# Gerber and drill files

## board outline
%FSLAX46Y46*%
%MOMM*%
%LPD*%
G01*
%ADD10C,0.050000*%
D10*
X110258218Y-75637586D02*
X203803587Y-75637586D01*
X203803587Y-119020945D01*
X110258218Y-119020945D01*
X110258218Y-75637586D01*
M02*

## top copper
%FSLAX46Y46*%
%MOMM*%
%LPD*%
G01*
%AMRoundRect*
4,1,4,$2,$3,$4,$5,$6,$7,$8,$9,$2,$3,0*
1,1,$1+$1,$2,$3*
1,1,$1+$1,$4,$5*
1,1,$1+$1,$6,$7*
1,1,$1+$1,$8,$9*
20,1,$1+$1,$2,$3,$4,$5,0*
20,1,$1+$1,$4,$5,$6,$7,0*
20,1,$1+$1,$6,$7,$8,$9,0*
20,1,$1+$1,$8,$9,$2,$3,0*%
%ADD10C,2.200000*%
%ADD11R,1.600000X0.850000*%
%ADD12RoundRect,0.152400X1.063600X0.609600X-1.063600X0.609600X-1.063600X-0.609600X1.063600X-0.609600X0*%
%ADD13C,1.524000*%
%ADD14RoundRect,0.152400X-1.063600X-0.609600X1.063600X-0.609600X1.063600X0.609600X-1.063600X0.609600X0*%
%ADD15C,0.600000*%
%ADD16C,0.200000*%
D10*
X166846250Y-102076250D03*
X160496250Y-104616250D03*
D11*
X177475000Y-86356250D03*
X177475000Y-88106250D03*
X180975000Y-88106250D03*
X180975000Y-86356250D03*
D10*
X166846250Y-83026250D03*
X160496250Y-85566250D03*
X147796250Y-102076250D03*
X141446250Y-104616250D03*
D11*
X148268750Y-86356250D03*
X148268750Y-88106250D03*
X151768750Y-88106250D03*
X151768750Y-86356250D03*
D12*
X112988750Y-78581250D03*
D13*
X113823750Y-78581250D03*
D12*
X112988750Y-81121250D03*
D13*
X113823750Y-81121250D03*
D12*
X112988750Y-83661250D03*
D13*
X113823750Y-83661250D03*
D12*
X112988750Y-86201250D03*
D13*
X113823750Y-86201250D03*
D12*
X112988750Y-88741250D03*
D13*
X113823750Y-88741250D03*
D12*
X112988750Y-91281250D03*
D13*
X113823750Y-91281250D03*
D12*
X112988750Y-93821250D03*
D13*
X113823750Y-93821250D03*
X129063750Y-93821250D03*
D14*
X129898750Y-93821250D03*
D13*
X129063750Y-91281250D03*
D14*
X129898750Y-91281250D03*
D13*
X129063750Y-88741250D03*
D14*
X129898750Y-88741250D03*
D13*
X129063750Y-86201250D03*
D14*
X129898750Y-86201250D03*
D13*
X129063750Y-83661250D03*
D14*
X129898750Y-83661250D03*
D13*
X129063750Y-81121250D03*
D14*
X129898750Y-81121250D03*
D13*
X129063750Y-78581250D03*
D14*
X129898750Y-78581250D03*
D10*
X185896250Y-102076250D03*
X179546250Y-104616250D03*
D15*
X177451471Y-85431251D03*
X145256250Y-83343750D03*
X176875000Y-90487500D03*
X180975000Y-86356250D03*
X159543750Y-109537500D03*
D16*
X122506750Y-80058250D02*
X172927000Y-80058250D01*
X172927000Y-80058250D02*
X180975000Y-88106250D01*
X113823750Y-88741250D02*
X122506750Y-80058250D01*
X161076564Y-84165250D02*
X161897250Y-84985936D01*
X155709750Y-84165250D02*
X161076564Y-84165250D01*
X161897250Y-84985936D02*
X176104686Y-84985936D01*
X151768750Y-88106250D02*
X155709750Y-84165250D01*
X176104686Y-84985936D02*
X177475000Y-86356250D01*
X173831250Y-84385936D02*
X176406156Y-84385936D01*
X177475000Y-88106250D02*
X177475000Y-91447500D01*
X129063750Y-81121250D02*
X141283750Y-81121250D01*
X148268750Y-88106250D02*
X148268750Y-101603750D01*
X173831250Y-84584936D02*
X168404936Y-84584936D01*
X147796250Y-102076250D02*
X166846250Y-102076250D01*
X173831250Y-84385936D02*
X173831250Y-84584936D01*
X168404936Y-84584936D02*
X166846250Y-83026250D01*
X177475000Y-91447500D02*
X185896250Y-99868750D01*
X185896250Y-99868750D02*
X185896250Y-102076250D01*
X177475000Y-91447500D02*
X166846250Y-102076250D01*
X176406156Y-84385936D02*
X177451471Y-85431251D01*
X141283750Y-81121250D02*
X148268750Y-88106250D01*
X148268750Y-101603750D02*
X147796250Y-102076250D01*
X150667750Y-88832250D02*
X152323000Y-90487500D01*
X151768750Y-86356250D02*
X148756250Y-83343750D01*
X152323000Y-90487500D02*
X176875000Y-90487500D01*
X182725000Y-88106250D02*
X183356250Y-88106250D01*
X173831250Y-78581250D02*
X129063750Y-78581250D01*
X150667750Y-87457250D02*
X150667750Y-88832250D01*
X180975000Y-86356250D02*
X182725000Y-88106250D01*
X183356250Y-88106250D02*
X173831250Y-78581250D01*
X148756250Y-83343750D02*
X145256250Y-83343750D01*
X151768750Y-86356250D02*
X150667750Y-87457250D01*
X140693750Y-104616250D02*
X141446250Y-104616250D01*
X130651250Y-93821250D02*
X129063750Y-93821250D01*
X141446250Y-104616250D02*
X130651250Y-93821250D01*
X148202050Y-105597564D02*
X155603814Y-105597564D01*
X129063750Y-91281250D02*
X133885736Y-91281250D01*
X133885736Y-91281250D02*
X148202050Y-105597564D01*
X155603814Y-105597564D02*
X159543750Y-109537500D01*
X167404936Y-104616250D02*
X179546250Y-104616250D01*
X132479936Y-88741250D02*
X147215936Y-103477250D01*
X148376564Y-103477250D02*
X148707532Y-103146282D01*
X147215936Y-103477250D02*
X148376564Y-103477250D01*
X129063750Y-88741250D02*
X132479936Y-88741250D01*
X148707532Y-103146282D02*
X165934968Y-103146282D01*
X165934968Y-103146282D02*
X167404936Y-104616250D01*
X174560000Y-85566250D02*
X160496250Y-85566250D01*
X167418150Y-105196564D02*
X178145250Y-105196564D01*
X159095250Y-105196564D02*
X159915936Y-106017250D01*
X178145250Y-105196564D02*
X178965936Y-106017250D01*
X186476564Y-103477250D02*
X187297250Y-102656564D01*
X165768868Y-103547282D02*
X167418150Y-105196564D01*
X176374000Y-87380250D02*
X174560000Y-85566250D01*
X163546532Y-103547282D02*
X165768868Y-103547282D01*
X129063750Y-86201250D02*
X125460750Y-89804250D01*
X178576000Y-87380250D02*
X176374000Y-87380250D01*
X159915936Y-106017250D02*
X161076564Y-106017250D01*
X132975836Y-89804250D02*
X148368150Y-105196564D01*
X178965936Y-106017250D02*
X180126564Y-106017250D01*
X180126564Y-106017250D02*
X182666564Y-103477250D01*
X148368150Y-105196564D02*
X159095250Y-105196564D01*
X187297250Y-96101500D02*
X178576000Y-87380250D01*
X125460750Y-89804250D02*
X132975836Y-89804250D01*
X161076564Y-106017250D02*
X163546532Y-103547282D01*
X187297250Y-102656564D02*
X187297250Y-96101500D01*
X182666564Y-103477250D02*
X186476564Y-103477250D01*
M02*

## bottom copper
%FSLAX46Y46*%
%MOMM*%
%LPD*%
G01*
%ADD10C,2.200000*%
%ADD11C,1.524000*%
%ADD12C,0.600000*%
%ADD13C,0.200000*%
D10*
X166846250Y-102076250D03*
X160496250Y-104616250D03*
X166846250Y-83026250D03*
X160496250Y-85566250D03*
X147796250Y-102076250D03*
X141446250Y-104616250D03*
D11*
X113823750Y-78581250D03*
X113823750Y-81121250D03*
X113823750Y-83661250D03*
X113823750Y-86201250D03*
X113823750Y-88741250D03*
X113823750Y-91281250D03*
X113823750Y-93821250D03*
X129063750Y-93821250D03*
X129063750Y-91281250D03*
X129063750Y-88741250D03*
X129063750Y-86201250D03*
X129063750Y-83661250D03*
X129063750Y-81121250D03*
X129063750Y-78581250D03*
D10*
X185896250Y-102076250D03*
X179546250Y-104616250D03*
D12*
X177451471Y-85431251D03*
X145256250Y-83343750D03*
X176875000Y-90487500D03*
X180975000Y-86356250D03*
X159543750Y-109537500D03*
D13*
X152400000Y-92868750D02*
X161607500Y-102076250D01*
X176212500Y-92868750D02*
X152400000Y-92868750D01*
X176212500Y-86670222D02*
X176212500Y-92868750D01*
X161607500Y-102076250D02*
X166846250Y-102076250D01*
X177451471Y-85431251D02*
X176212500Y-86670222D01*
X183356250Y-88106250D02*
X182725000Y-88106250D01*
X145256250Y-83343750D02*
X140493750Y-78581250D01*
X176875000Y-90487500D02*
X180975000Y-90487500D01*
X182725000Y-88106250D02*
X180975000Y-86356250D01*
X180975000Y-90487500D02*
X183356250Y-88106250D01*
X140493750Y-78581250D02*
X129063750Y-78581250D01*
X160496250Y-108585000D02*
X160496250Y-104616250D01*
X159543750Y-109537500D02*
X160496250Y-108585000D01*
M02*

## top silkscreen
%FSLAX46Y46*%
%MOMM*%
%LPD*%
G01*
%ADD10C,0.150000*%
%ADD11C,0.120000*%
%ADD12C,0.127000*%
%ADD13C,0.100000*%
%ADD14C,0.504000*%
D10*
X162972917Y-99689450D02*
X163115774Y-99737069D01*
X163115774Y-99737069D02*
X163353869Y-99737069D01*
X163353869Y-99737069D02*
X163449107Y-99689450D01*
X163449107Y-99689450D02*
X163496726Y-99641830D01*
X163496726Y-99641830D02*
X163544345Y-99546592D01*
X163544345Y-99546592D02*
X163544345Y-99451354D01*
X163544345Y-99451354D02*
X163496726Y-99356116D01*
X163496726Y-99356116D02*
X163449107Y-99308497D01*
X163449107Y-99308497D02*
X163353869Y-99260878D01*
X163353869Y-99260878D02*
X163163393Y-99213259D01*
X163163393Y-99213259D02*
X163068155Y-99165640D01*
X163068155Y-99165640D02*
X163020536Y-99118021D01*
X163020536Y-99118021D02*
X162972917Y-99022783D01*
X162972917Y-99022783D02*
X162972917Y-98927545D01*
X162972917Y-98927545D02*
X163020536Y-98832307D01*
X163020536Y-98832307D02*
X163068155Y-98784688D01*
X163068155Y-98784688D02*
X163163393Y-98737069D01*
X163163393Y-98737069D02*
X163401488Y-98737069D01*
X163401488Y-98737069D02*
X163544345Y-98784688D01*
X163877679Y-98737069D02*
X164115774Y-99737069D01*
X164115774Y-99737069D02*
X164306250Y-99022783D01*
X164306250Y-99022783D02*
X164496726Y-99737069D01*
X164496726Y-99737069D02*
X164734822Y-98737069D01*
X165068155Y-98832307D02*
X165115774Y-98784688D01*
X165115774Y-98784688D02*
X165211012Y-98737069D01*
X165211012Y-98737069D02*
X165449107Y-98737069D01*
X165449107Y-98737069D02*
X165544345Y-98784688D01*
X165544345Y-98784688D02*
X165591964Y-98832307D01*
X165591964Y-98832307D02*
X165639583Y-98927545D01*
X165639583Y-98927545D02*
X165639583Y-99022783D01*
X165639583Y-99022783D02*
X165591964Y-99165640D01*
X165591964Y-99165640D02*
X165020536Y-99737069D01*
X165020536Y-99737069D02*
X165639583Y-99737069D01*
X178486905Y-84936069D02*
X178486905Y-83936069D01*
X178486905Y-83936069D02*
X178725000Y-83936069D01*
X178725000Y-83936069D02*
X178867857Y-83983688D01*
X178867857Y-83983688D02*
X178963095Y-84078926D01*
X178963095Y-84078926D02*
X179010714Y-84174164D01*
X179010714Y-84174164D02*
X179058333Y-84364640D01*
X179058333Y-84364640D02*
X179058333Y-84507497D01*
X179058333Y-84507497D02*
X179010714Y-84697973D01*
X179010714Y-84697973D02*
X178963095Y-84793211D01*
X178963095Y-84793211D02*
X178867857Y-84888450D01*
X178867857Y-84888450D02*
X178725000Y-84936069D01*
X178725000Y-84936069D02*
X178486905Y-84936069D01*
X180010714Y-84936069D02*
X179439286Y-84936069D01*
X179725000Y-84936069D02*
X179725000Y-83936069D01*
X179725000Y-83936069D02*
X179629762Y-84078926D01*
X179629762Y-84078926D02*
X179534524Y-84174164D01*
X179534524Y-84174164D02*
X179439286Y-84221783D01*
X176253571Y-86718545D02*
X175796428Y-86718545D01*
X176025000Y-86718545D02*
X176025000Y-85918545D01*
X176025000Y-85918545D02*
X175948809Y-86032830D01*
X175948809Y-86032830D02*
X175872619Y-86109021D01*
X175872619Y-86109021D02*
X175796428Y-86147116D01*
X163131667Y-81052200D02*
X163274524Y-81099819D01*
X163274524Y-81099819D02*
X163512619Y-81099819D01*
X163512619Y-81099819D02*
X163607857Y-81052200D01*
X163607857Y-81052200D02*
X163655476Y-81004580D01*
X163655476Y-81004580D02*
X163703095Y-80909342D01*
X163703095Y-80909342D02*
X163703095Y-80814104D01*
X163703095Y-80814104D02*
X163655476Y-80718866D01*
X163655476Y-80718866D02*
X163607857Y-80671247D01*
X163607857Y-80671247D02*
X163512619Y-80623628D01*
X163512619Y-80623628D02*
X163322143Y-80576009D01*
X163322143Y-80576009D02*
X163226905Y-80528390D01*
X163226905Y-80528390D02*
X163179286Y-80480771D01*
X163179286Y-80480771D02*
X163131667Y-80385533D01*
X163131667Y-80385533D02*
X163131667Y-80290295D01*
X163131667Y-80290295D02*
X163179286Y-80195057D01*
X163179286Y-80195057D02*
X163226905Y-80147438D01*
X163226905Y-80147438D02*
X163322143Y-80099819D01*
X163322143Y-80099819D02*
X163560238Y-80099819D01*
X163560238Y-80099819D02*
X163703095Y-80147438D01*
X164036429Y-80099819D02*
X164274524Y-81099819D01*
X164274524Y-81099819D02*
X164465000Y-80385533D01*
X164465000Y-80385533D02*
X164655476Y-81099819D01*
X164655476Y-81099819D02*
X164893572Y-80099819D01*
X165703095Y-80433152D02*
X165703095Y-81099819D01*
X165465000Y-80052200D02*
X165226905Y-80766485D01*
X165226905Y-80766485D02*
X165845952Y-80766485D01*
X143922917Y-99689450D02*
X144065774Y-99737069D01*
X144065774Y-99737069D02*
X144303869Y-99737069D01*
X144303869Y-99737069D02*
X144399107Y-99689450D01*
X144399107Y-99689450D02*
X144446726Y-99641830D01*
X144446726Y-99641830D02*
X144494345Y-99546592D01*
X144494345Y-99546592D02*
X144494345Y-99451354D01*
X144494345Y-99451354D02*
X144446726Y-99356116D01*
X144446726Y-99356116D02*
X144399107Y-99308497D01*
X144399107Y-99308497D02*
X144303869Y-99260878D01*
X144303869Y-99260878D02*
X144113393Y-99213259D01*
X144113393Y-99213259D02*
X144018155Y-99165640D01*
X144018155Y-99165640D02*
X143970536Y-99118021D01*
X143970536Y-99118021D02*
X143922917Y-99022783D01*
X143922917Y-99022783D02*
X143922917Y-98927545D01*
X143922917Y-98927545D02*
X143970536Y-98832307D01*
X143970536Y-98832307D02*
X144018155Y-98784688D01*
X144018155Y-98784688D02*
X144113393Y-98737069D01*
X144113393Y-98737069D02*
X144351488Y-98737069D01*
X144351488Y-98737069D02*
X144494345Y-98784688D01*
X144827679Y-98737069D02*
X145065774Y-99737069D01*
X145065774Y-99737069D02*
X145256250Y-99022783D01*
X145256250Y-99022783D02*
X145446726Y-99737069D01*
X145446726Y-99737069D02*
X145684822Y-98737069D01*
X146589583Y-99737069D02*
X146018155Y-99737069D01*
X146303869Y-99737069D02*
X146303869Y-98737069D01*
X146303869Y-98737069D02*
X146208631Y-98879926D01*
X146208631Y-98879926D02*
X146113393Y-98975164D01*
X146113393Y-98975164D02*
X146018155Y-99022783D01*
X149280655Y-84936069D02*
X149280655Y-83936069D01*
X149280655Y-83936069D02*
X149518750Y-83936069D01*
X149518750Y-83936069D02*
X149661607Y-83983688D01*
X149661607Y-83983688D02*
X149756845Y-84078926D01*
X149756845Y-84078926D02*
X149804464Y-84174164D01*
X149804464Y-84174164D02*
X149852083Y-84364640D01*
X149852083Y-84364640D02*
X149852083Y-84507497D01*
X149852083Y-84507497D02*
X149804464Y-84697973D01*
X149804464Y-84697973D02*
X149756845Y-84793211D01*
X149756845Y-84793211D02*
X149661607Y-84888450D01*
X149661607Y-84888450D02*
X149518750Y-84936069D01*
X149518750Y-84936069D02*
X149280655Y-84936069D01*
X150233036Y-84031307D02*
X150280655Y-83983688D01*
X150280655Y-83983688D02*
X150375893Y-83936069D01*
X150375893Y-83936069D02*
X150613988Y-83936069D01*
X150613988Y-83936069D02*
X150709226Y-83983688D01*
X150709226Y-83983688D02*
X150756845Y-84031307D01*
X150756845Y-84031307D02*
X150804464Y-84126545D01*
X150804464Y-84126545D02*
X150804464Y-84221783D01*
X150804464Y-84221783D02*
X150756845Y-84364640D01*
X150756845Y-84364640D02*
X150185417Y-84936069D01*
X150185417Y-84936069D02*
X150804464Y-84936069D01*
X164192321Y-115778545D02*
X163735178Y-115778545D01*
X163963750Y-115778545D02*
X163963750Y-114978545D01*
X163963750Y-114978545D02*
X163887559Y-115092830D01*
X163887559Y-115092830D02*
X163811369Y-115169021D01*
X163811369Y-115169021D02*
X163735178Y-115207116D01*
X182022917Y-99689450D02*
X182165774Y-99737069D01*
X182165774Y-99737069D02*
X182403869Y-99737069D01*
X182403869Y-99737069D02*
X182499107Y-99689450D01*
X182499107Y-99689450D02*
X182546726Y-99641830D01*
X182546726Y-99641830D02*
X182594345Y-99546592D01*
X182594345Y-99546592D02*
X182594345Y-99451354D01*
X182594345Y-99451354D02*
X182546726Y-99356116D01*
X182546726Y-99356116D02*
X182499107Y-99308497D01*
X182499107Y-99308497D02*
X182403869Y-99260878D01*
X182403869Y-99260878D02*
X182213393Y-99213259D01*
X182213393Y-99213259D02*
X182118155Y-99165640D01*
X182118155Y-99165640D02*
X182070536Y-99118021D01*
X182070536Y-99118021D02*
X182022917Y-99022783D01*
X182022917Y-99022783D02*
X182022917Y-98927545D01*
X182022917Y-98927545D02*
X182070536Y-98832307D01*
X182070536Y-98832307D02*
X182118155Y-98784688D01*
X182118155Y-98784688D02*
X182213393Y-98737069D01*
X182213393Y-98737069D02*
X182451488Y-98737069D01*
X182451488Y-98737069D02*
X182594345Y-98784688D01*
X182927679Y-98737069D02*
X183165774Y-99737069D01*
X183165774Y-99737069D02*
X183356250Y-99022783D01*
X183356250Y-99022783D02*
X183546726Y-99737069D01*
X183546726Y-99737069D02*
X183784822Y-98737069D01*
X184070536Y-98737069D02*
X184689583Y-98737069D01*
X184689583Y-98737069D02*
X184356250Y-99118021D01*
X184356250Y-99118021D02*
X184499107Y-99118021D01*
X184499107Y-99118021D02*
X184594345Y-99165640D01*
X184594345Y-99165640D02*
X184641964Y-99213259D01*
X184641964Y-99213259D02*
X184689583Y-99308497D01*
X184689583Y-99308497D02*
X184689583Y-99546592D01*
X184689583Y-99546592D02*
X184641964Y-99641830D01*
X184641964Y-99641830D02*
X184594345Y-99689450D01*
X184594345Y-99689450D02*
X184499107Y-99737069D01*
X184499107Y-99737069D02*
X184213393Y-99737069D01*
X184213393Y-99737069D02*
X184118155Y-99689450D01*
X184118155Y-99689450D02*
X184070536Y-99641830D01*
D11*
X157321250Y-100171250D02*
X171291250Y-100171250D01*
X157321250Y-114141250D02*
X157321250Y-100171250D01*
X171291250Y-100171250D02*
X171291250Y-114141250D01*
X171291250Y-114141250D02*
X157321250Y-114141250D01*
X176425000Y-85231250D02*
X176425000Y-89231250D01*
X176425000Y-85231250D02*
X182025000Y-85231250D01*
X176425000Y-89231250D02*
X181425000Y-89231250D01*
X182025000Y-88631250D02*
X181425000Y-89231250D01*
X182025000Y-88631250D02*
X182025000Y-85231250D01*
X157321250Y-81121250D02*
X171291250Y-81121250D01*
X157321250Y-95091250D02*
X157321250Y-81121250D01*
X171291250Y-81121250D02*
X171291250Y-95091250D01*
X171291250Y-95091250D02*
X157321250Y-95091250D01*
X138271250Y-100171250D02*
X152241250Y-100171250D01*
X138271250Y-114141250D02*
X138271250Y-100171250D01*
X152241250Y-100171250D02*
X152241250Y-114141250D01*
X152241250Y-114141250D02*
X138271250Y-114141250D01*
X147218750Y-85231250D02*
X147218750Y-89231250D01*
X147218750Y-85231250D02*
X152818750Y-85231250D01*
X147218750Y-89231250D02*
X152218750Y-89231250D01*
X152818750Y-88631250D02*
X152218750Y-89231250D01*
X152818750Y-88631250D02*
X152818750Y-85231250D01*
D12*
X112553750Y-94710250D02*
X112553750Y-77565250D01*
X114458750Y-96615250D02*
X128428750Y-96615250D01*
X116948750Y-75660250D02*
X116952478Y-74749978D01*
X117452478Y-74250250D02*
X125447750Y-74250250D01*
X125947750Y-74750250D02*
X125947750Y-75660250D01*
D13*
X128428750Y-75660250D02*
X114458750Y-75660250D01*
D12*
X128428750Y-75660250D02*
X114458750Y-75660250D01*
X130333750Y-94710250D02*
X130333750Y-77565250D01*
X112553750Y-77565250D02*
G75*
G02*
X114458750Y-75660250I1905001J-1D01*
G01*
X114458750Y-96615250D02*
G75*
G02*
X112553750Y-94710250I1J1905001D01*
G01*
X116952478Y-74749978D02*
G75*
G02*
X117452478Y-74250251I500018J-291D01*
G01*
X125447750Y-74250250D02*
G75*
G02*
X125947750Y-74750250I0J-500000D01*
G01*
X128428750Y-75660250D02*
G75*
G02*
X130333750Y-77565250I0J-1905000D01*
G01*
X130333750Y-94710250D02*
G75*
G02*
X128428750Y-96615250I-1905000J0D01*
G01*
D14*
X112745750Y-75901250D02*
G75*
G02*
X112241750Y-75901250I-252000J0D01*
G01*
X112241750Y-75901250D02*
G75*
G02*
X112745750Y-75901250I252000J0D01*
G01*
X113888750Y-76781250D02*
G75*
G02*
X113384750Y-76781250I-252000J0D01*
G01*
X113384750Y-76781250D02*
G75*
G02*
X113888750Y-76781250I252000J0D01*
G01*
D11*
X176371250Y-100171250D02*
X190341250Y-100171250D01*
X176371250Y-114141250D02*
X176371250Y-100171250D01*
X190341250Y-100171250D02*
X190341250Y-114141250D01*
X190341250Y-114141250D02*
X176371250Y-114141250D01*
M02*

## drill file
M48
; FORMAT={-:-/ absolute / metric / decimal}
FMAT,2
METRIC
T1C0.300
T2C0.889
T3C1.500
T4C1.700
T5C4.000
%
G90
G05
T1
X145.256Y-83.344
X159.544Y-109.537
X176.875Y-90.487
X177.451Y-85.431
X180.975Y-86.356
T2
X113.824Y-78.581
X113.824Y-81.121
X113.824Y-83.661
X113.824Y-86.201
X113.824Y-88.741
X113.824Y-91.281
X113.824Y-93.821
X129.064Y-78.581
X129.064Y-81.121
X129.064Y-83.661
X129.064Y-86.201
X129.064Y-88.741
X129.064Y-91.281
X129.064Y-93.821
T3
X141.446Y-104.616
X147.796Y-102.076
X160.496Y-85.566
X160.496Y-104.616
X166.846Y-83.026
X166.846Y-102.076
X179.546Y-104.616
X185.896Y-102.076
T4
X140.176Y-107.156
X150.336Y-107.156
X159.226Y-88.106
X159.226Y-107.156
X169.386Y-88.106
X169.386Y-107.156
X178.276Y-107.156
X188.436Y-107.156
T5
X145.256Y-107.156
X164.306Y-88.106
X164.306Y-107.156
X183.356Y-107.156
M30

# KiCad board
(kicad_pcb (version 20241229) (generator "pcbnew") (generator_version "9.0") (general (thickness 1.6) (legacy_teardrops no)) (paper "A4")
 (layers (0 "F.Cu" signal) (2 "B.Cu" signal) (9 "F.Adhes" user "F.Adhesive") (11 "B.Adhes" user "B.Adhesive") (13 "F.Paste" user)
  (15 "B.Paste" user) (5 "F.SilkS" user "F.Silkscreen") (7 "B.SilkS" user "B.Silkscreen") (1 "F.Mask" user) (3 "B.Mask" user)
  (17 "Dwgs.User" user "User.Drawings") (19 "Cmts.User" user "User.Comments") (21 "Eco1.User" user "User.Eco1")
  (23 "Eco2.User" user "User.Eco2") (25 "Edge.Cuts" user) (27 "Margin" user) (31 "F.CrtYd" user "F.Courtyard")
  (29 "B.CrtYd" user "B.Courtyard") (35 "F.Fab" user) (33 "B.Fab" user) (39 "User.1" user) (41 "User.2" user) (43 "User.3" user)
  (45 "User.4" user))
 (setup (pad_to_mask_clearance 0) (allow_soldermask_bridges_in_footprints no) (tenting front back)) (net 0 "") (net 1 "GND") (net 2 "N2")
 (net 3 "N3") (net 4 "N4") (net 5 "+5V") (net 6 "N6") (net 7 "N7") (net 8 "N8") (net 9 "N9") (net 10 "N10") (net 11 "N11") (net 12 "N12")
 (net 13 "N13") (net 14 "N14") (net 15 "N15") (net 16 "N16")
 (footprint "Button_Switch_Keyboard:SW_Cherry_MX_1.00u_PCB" (layer "F.Cu") (at 166.84625 102.07625)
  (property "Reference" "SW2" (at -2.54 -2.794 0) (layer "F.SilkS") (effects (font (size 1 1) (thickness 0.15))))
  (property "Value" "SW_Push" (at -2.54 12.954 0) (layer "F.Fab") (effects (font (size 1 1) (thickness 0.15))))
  (fp_line (start -9.525 -1.905) (end 4.445 -1.905) (stroke (width 0.12) (type solid)) (layer "F.SilkS"))
  (fp_line (start -9.525 12.065) (end -9.525 -1.905) (stroke (width 0.12) (type solid)) (layer "F.SilkS"))
  (fp_line (start 4.445 -1.905) (end 4.445 12.065) (stroke (width 0.12) (type solid)) (layer "F.SilkS"))
  (fp_line (start 4.445 12.065) (end -9.525 12.065) (stroke (width 0.12) (type solid)) (layer "F.SilkS"))
  (pad "" np_thru_hole circle (at -7.62 5.08) (size 1.7 1.7) (drill 1.7) (layers "*.Cu" "*.Mask"))
  (pad "" np_thru_hole circle (at -2.54 5.08) (size 4 4) (drill 4) (layers "*.Cu" "*.Mask"))
  (pad "" np_thru_hole circle (at 2.54 5.08) (size 1.7 1.7) (drill 1.7) (layers "*.Cu" "*.Mask"))
  (pad "1" thru_hole circle (at 0 0) (size 2.2 2.2) (drill 1.5) (layers "*.Cu" "*.Mask") (remove_unused_layers no) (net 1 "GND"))
  (pad "2" thru_hole circle (at -6.35 2.54) (size 2.2 2.2) (drill 1.5) (layers "*.Cu" "*.Mask") (remove_unused_layers no) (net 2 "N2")))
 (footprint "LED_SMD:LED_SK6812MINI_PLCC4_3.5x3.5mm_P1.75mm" (layer "F.Cu") (at 179.225 87.23125)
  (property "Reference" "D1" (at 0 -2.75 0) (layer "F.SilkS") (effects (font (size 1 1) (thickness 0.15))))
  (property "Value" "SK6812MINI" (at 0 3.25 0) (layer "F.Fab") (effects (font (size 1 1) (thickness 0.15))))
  (fp_line (start -2.8 -2) (end -2.8 2) (stroke (width 0.12) (type default)) (layer "F.SilkS"))
  (fp_line (start -2.8 -2) (end 2.8 -2) (stroke (width 0.12) (type solid)) (layer "F.SilkS"))
  (fp_line (start -2.8 2) (end 2.2 2) (stroke (width 0.12) (type solid)) (layer "F.SilkS"))
  (fp_line (start 2.8 1.4) (end 2.2 2) (stroke (width 0.12) (type default)) (layer "F.SilkS"))
  (fp_line (start 2.8 1.4) (end 2.8 -2) (stroke (width 0.12) (type solid)) (layer "F.SilkS"))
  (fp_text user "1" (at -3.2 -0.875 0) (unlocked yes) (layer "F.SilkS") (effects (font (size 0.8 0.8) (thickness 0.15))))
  (pad "1" smd rect (at -1.75 -0.875) (size 1.6 0.85) (layers "F.Cu" "F.Mask" "F.Paste") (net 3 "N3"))
  (pad "2" smd rect (at -1.75 0.875) (size 1.6 0.85) (layers "F.Cu" "F.Mask" "F.Paste") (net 1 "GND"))
  (pad "3" smd rect (at 1.75 0.875) (size 1.6 0.85) (layers "F.Cu" "F.Mask" "F.Paste") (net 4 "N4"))
  (pad "4" smd rect (at 1.75 -0.875) (size 1.6 0.85) (layers "F.Cu" "F.Mask" "F.Paste") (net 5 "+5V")))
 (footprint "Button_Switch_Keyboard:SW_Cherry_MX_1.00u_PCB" (layer "F.Cu") (at 166.84625 83.02625)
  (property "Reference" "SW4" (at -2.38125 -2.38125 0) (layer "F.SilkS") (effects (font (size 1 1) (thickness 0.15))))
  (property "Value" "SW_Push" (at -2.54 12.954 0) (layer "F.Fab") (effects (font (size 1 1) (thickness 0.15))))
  (fp_line (start -9.525 -1.905) (end 4.445 -1.905) (stroke (width 0.12) (type solid)) (layer "F.SilkS"))
  (fp_line (start -9.525 12.065) (end -9.525 -1.905) (stroke (width 0.12) (type solid)) (layer "F.SilkS"))
  (fp_line (start 4.445 -1.905) (end 4.445 12.065) (stroke (width 0.12) (type solid)) (layer "F.SilkS"))
  (fp_line (start 4.445 12.065) (end -9.525 12.065) (stroke (width 0.12) (type solid)) (layer "F.SilkS"))
  (pad "" np_thru_hole circle (at -7.62 5.08) (size 1.7 1.7) (drill 1.7) (layers "*.Cu" "*.Mask"))
  (pad "" np_thru_hole circle (at -2.54 5.08) (size 4 4) (drill 4) (layers "*.Cu" "*.Mask"))
  (pad "" np_thru_hole circle (at 2.54 5.08) (size 1.7 1.7) (drill 1.7) (layers "*.Cu" "*.Mask"))
  (pad "1" thru_hole circle (at 0 0) (size 2.2 2.2) (drill 1.5) (layers "*.Cu" "*.Mask") (remove_unused_layers no) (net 1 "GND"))
  (pad "2" thru_hole circle (at -6.35 2.54) (size 2.2 2.2) (drill 1.5) (layers "*.Cu" "*.Mask") (remove_unused_layers no) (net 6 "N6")))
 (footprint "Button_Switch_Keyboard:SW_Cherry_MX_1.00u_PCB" (layer "F.Cu") (at 147.79625 102.07625)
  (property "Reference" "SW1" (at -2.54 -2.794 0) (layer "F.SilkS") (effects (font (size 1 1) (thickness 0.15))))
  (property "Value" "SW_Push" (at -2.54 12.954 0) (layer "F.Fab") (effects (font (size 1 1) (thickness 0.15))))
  (fp_line (start -9.525 -1.905) (end 4.445 -1.905) (stroke (width 0.12) (type solid)) (layer "F.SilkS"))
  (fp_line (start -9.525 12.065) (end -9.525 -1.905) (stroke (width 0.12) (type solid)) (layer "F.SilkS"))
  (fp_line (start 4.445 -1.905) (end 4.445 12.065) (stroke (width 0.12) (type solid)) (layer "F.SilkS"))
  (fp_line (start 4.445 12.065) (end -9.525 12.065) (stroke (width 0.12) (type solid)) (layer "F.SilkS"))
  (pad "" np_thru_hole circle (at -7.62 5.08) (size 1.7 1.7) (drill 1.7) (layers "*.Cu" "*.Mask"))
  (pad "" np_thru_hole circle (at -2.54 5.08) (size 4 4) (drill 4) (layers "*.Cu" "*.Mask"))
  (pad "" np_thru_hole circle (at 2.54 5.08) (size 1.7 1.7) (drill 1.7) (layers "*.Cu" "*.Mask"))
  (pad "1" thru_hole circle (at 0 0) (size 2.2 2.2) (drill 1.5) (layers "*.Cu" "*.Mask") (remove_unused_layers no) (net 1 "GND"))
  (pad "2" thru_hole circle (at -6.35 2.54) (size 2.2 2.2) (drill 1.5) (layers "*.Cu" "*.Mask") (remove_unused_layers no) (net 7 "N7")))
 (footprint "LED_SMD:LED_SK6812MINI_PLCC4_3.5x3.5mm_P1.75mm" (layer "F.Cu") (at 150.01875 87.23125)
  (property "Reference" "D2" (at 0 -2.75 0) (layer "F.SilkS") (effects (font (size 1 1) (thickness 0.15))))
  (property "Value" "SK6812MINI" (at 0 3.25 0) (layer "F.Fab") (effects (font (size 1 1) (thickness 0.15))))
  (fp_line (start -2.8 -2) (end -2.8 2) (stroke (width 0.12) (type default)) (layer "F.SilkS"))
  (fp_line (start -2.8 -2) (end 2.8 -2) (stroke (width 0.12) (type solid)) (layer "F.SilkS"))
  (fp_line (start -2.8 2) (end 2.2 2) (stroke (width 0.12) (type solid)) (layer "F.SilkS"))
  (fp_line (start 2.8 1.4) (end 2.2 2) (stroke (width 0.12) (type default)) (layer "F.SilkS"))
  (fp_line (start 2.8 1.4) (end 2.8 -2) (stroke (width 0.12) (type solid)) (layer "F.SilkS"))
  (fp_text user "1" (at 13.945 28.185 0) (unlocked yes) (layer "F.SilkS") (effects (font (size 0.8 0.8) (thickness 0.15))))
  (pad "1" smd rect (at -1.75 -0.875) (size 1.6 0.85) (layers "F.Cu" "F.Mask" "F.Paste") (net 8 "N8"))
  (pad "2" smd rect (at -1.75 0.875) (size 1.6 0.85) (layers "F.Cu" "F.Mask" "F.Paste") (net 1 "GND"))
  (pad "3" smd rect (at 1.75 0.875) (size 1.6 0.85) (layers "F.Cu" "F.Mask" "F.Paste") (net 3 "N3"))
  (pad "4" smd rect (at 1.75 -0.875) (size 1.6 0.85) (layers "F.Cu" "F.Mask" "F.Paste") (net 5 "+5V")))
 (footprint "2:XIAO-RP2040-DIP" (layer "F.Cu") (at 121.44375 86.20125)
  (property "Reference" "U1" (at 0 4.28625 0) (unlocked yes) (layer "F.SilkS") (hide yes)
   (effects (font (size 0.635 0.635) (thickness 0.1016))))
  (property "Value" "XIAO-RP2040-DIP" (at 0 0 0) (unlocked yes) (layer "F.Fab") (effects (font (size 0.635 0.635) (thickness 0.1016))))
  (fp_line (start -8.89 8.509) (end -8.89 -8.636) (stroke (width 0.127) (type solid)) (layer "F.SilkS"))
  (fp_line (start -6.985 10.414) (end 6.985 10.414) (stroke (width 0.127) (type solid)) (layer "F.SilkS"))
  (fp_line (start -4.495 -10.541) (end -4.491272 -11.451272) (stroke (width 0.127) (type solid)) (layer "F.SilkS"))
  (fp_line (start -3.991272 -11.951) (end 4.004 -11.951) (stroke (width 0.127) (type solid)) (layer "F.SilkS"))
  (fp_line (start 4.504 -11.451) (end 4.504 -10.541) (stroke (width 0.127) (type solid)) (layer "F.SilkS"))
  (fp_line (start 6.985 -10.541) (end -6.985 -10.541) (stroke (width 0.1) (type solid)) (layer "F.SilkS"))
  (fp_line (start 6.985 -10.541) (end -6.985 -10.541) (stroke (width 0.127) (type solid)) (layer "F.SilkS"))
  (fp_line (start 8.89 8.509) (end 8.89 -8.636) (stroke (width 0.127) (type solid)) (layer "F.SilkS"))
  (fp_arc (start -8.89 -8.636) (mid -8.332038 -9.983038) (end -6.985 -10.541) (stroke (width 0.127) (type solid)) (layer "F.SilkS"))
  (fp_arc (start -6.985 10.414) (mid -8.332038 9.856038) (end -8.89 8.509) (stroke (width 0.127) (type solid)) (layer "F.SilkS"))
  (fp_arc (start -4.491272 -11.451272) (mid -4.344728 -11.80464) (end -3.991272 -11.951) (stroke (width 0.127) (type default))
   (layer "F.SilkS"))
  (fp_arc (start 4.004 -11.951) (mid 4.357553 -11.804553) (end 4.504 -11.451) (stroke (width 0.127) (type default)) (layer "F.SilkS"))
  (fp_arc (start 6.985 -10.541) (mid 8.332038 -9.983038) (end 8.89 -8.636) (stroke (width 0.127) (type solid)) (layer "F.SilkS"))
  (fp_arc (start 8.89 8.509) (mid 8.332038 9.856038) (end 6.985 10.414) (stroke (width 0.127) (type solid)) (layer "F.SilkS"))
  (fp_circle (center -8.95 -10.3) (end -8.95 -10.554) (stroke (width 0.5) (type solid)) (fill yes) (layer "F.SilkS"))
  (fp_circle (center -7.807 -9.42) (end -7.807 -9.674) (stroke (width 0.5) (type solid)) (fill yes) (layer "F.SilkS"))
  (pad "1" smd roundrect (at -8.455 -7.62 180) (size 2.432 1.524) (layers "F.Cu" "F.Mask") (roundrect_rratio 0.1) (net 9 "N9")
   (thermal_bridge_angle 45))
  (pad "1" thru_hole circle (at -7.62 -7.62 180) (size 1.524 1.524) (drill 0.889) (layers "*.Cu" "*.Mask") (remove_unused_layers no)
   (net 9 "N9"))
  (pad "2" smd roundrect (at -8.455 -5.08 180) (size 2.432 1.524) (layers "F.Cu" "F.Mask") (roundrect_rratio 0.1) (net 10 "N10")
   (thermal_bridge_angle 45))
  (pad "2" thru_hole circle (at -7.62 -5.08 180) (size 1.524 1.524) (drill 0.889) (layers "*.Cu" "*.Mask") (remove_unused_layers no)
   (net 10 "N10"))
  (pad "3" smd roundrect (at -8.455 -2.54 180) (size 2.432 1.524) (layers "F.Cu" "F.Mask") (roundrect_rratio 0.1) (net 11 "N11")
   (thermal_bridge_angle 45))
  (pad "3" thru_hole circle (at -7.62 -2.54 180) (size 1.524 1.524) (drill 0.889) (layers "*.Cu" "*.Mask") (remove_unused_layers no)
   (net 11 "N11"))
  (pad "4" smd roundrect (at -8.455 0 180) (size 2.432 1.524) (layers "F.Cu" "F.Mask") (roundrect_rratio 0.1) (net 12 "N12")
   (thermal_bridge_angle 45))
  (pad "4" thru_hole circle (at -7.62 0 180) (size 1.524 1.524) (drill 0.889) (layers "*.Cu" "*.Mask") (remove_unused_layers no)
   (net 12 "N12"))
  (pad "5" smd roundrect (at -8.455 2.54 180) (size 2.432 1.524) (layers "F.Cu" "F.Mask") (roundrect_rratio 0.1) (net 4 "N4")
   (thermal_bridge_angle 45))
  (pad "5" thru_hole circle (at -7.62 2.54 180) (size 1.524 1.524) (drill 0.889) (layers "*.Cu" "*.Mask") (remove_unused_layers no)
   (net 4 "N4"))
  (pad "6" smd roundrect (at -8.455 5.08 180) (size 2.432 1.524) (layers "F.Cu" "F.Mask") (roundrect_rratio 0.1) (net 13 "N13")
   (thermal_bridge_angle 45))
  (pad "6" thru_hole circle (at -7.62 5.08 180) (size 1.524 1.524) (drill 0.889) (layers "*.Cu" "*.Mask") (remove_unused_layers no)
   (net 13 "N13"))
  (pad "7" smd roundrect (at -8.455 7.62 180) (size 2.432 1.524) (layers "F.Cu" "F.Mask") (roundrect_rratio 0.1) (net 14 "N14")
   (thermal_bridge_angle 45))
  (pad "7" thru_hole circle (at -7.62 7.62 180) (size 1.524 1.524) (drill 0.889) (layers "*.Cu" "*.Mask") (remove_unused_layers no)
   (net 14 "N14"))
  (pad "8" thru_hole circle (at 7.62 7.62) (size 1.524 1.524) (drill 0.889) (layers "*.Cu" "*.Mask") (remove_unused_layers no) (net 7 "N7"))
  (pad "8" smd roundrect (at 8.455 7.62) (size 2.432 1.524) (layers "F.Cu" "F.Mask") (roundrect_rratio 0.1) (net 7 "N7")
   (thermal_bridge_angle 45))
  (pad "9" thru_hole circle (at 7.62 5.08) (size 1.524 1.524) (drill 0.889) (layers "*.Cu" "*.Mask") (remove_unused_layers no) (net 2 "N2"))
  (pad "9" smd roundrect (at 8.455 5.08) (size 2.432 1.524) (layers "F.Cu" "F.Mask") (roundrect_rratio 0.1) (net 2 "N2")
   (thermal_bridge_angle 45))
  (pad "10" thru_hole circle (at 7.62 2.54) (size 1.524 1.524) (drill 0.889) (layers "*.Cu" "*.Mask") (remove_unused_layers no)
   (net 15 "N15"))
  (pad "10" smd roundrect (at 8.455 2.54) (size 2.432 1.524) (layers "F.Cu" "F.Mask") (roundrect_rratio 0.1) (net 15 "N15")
   (thermal_bridge_angle 45))
  (pad "11" thru_hole circle (at 7.62 0) (size 1.524 1.524) (drill 0.889) (layers "*.Cu" "*.Mask") (remove_unused_layers no) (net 6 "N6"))
  (pad "11" smd roundrect (at 8.455 0) (size 2.432 1.524) (layers "F.Cu" "F.Mask") (roundrect_rratio 0.1) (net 6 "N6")
   (thermal_bridge_angle 45))
  (pad "12" thru_hole circle (at 7.62 -2.54) (size 1.524 1.524) (drill 0.889) (layers "*.Cu" "*.Mask") (remove_unused_layers no)
   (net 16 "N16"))
  (pad "12" smd roundrect (at 8.455 -2.54) (size 2.432 1.524) (layers "F.Cu" "F.Mask") (roundrect_rratio 0.1) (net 16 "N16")
   (thermal_bridge_angle 45))
  (pad "13" thru_hole circle (at 7.62 -5.08) (size 1.524 1.524) (drill 0.889) (layers "*.Cu" "*.Mask") (remove_unused_layers no)
   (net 1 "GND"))
  (pad "13" smd roundrect (at 8.455 -5.08) (size 2.432 1.524) (layers "F.Cu" "F.Mask") (roundrect_rratio 0.1) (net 1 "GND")
   (thermal_bridge_angle 45))
  (pad "14" thru_hole circle (at 7.62 -7.62) (size 1.524 1.524) (drill 0.889) (layers "*.Cu" "*.Mask") (remove_unused_layers no)
   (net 5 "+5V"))
  (pad "14" smd roundrect (at 8.455 -7.62) (size 2.432 1.524) (layers "F.Cu" "F.Mask") (roundrect_rratio 0.1) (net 5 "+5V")
   (thermal_bridge_angle 45)))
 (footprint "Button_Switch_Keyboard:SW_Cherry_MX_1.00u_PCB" (layer "F.Cu") (at 185.89625 102.07625)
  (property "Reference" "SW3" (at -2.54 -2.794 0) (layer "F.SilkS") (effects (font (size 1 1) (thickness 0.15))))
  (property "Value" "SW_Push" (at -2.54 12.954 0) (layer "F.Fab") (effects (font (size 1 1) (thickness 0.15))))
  (fp_line (start -9.525 -1.905) (end 4.445 -1.905) (stroke (width 0.12) (type solid)) (layer "F.SilkS"))
  (fp_line (start -9.525 12.065) (end -9.525 -1.905) (stroke (width 0.12) (type solid)) (layer "F.SilkS"))
  (fp_line (start 4.445 -1.905) (end 4.445 12.065) (stroke (width 0.12) (type solid)) (layer "F.SilkS"))
  (fp_line (start 4.445 12.065) (end -9.525 12.065) (stroke (width 0.12) (type solid)) (layer "F.SilkS"))
  (pad "" np_thru_hole circle (at -7.62 5.08) (size 1.7 1.7) (drill 1.7) (layers "*.Cu" "*.Mask"))
  (pad "" np_thru_hole circle (at -2.54 5.08) (size 4 4) (drill 4) (layers "*.Cu" "*.Mask"))
  (pad "" np_thru_hole circle (at 2.54 5.08) (size 1.7 1.7) (drill 1.7) (layers "*.Cu" "*.Mask"))
  (pad "1" thru_hole circle (at 0 0) (size 2.2 2.2) (drill 1.5) (layers "*.Cu" "*.Mask") (remove_unused_layers no) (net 1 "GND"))
  (pad "2" thru_hole circle (at -6.35 2.54) (size 2.2 2.2) (drill 1.5) (layers "*.Cu" "*.Mask") (remove_unused_layers no) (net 15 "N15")))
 (gr_rect (start 110.258218 75.637586) (end 203.803587 119.020945) (stroke (width 0.05) (type default)) (fill no) (layer "Edge.Cuts"))
 (segment (start 122.50675 80.05825) (end 172.927 80.05825) (width 0.2) (layer "F.Cu") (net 4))
 (segment (start 172.927 80.05825) (end 180.975 88.10625) (width 0.2) (layer "F.Cu") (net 4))
 (segment (start 113.82375 88.74125) (end 122.50675 80.05825) (width 0.2) (layer "F.Cu") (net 4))
 (segment (start 161.076564 84.16525) (end 161.89725 84.985936) (width 0.2) (layer "F.Cu") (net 3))
 (segment (start 155.70975 84.16525) (end 161.076564 84.16525) (width 0.2) (layer "F.Cu") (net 3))
 (segment (start 161.89725 84.985936) (end 176.104686 84.985936) (width 0.2) (layer "F.Cu") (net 3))
 (segment (start 151.76875 88.10625) (end 155.70975 84.16525) (width 0.2) (layer "F.Cu") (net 3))
 (segment (start 176.104686 84.985936) (end 177.475 86.35625) (width 0.2) (layer "F.Cu") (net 3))
 (segment (start 173.83125 84.385936) (end 176.406156 84.385936) (width 0.2) (layer "F.Cu") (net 1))
 (segment (start 177.475 88.10625) (end 177.475 91.4475) (width 0.2) (layer "F.Cu") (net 1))
 (segment (start 129.06375 81.12125) (end 141.28375 81.12125) (width 0.2) (layer "F.Cu") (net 1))
 (segment (start 148.26875 88.10625) (end 148.26875 101.60375) (width 0.2) (layer "F.Cu") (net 1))
 (segment (start 173.83125 84.584936) (end 168.404936 84.584936) (width 0.2) (layer "F.Cu") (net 1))
 (segment (start 147.79625 102.07625) (end 166.84625 102.07625) (width 0.2) (layer "F.Cu") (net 1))
 (segment (start 173.83125 84.385936) (end 173.83125 84.584936) (width 0.2) (layer "F.Cu") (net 1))
 (segment (start 168.404936 84.584936) (end 166.84625 83.02625) (width 0.2) (layer "F.Cu") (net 1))
 (segment (start 177.475 91.4475) (end 185.89625 99.86875) (width 0.2) (layer "F.Cu") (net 1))
 (segment (start 185.89625 99.86875) (end 185.89625 102.07625) (width 0.2) (layer "F.Cu") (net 1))
 (segment (start 177.475 91.4475) (end 166.84625 102.07625) (width 0.2) (layer "F.Cu") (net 1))
 (segment (start 176.406156 84.385936) (end 177.451471 85.431251) (width 0.2) (layer "F.Cu") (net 1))
 (segment (start 141.28375 81.12125) (end 148.26875 88.10625) (width 0.2) (layer "F.Cu") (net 1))
 (segment (start 148.26875 101.60375) (end 147.79625 102.07625) (width 0.2) (layer "F.Cu") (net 1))
 (via (at 177.451471 85.431251) (size 0.6) (drill 0.3) (layers "F.Cu" "B.Cu") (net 1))
 (segment (start 152.4 92.86875) (end 161.6075 102.07625) (width 0.2) (layer "B.Cu") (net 1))
 (segment (start 176.2125 92.86875) (end 152.4 92.86875) (width 0.2) (layer "B.Cu") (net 1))
 (segment (start 176.2125 86.670222) (end 176.2125 92.86875) (width 0.2) (layer "B.Cu") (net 1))
 (segment (start 161.6075 102.07625) (end 166.84625 102.07625) (width 0.2) (layer "B.Cu") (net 1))
 (segment (start 177.451471 85.431251) (end 176.2125 86.670222) (width 0.2) (layer "B.Cu") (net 1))
 (segment (start 150.66775 88.83225) (end 152.323 90.4875) (width 0.2) (layer "F.Cu") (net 5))
 (segment (start 151.76875 86.35625) (end 148.75625 83.34375) (width 0.2) (layer "F.Cu") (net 5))
 (segment (start 152.323 90.4875) (end 176.875 90.4875) (width 0.2) (layer "F.Cu") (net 5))
 (segment (start 182.725 88.10625) (end 183.35625 88.10625) (width 0.2) (layer "F.Cu") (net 5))
 (segment (start 173.83125 78.58125) (end 129.06375 78.58125) (width 0.2) (layer "F.Cu") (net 5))
 (segment (start 150.66775 87.45725) (end 150.66775 88.83225) (width 0.2) (layer "F.Cu") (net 5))
 (segment (start 180.975 86.35625) (end 182.725 88.10625) (width 0.2) (layer "F.Cu") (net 5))
 (segment (start 183.35625 88.10625) (end 173.83125 78.58125) (width 0.2) (layer "F.Cu") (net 5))
 (segment (start 148.75625 83.34375) (end 145.25625 83.34375) (width 0.2) (layer "F.Cu") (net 5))
 (segment (start 151.76875 86.35625) (end 150.66775 87.45725) (width 0.2) (layer "F.Cu") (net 5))
 (via (at 145.25625 83.34375) (size 0.6) (drill 0.3) (layers "F.Cu" "B.Cu") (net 5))
 (via (at 176.875 90.4875) (size 0.6) (drill 0.3) (layers "F.Cu" "B.Cu") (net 5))
 (via (at 180.975 86.35625) (size 0.6) (drill 0.3) (layers "F.Cu" "B.Cu") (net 5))
 (segment (start 183.35625 88.10625) (end 182.725 88.10625) (width 0.2) (layer "B.Cu") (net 5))
 (segment (start 145.25625 83.34375) (end 140.49375 78.58125) (width 0.2) (layer "B.Cu") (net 5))
 (segment (start 176.875 90.4875) (end 180.975 90.4875) (width 0.2) (layer "B.Cu") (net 5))
 (segment (start 182.725 88.10625) (end 180.975 86.35625) (width 0.2) (layer "B.Cu") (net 5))
 (segment (start 180.975 90.4875) (end 183.35625 88.10625) (width 0.2) (layer "B.Cu") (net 5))
 (segment (start 140.49375 78.58125) (end 129.06375 78.58125) (width 0.2) (layer "B.Cu") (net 5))
 (segment (start 140.69375 104.61625) (end 141.44625 104.61625) (width 0.2) (layer "F.Cu") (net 7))
 (segment (start 130.65125 93.82125) (end 129.06375 93.82125) (width 0.2) (layer "F.Cu") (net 7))
 (segment (start 141.44625 104.61625) (end 130.65125 93.82125) (width 0.2) (layer "F.Cu") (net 7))
 (segment (start 148.20205 105.597564) (end 155.603814 105.597564) (width 0.2) (layer "F.Cu") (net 2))
 (segment (start 129.06375 91.28125) (end 133.885736 91.28125) (width 0.2) (layer "F.Cu") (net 2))
 (segment (start 133.885736 91.28125) (end 148.20205 105.597564) (width 0.2) (layer "F.Cu") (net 2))
 (segment (start 155.603814 105.597564) (end 159.54375 109.5375) (width 0.2) (layer "F.Cu") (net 2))
 (via (at 159.54375 109.5375) (size 0.6) (drill 0.3) (layers "F.Cu" "B.Cu") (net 2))
 (segment (start 160.49625 108.585) (end 160.49625 104.61625) (width 0.2) (layer "B.Cu") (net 2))
 (segment (start 159.54375 109.5375) (end 160.49625 108.585) (width 0.2) (layer "B.Cu") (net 2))
 (segment (start 167.404936 104.61625) (end 179.54625 104.61625) (width 0.2) (layer "F.Cu") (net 15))
 (segment (start 132.479936 88.74125) (end 147.215936 103.47725) (width 0.2) (layer "F.Cu") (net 15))
 (segment (start 148.376564 103.47725) (end 148.707532 103.146282) (width 0.2) (layer "F.Cu") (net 15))
 (segment (start 147.215936 103.47725) (end 148.376564 103.47725) (width 0.2) (layer "F.Cu") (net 15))
 (segment (start 129.06375 88.74125) (end 132.479936 88.74125) (width 0.2) (layer "F.Cu") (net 15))
 (segment (start 148.707532 103.146282) (end 165.934968 103.146282) (width 0.2) (layer "F.Cu") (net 15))
 (segment (start 165.934968 103.146282) (end 167.404936 104.61625) (width 0.2) (layer "F.Cu") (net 15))
 (segment (start 174.56 85.56625) (end 160.49625 85.56625) (width 0.2) (layer "F.Cu") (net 6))
 (segment (start 167.41815 105.196564) (end 178.14525 105.196564) (width 0.2) (layer "F.Cu") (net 6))
 (segment (start 159.09525 105.196564) (end 159.915936 106.01725) (width 0.2) (layer "F.Cu") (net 6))
 (segment (start 178.14525 105.196564) (end 178.965936 106.01725) (width 0.2) (layer "F.Cu") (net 6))
 (segment (start 186.476564 103.47725) (end 187.29725 102.656564) (width 0.2) (layer "F.Cu") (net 6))
 (segment (start 165.768868 103.547282) (end 167.41815 105.196564) (width 0.2) (layer "F.Cu") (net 6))
 (segment (start 176.374 87.38025) (end 174.56 85.56625) (width 0.2) (layer "F.Cu") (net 6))
 (segment (start 163.546532 103.547282) (end 165.768868 103.547282) (width 0.2) (layer "F.Cu") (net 6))
 (segment (start 129.06375 86.20125) (end 125.46075 89.80425) (width 0.2) (layer "F.Cu") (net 6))
 (segment (start 178.576 87.38025) (end 176.374 87.38025) (width 0.2) (layer "F.Cu") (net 6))
 (segment (start 159.915936 106.01725) (end 161.076564 106.01725) (width 0.2) (layer "F.Cu") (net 6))
 (segment (start 132.975836 89.80425) (end 148.36815 105.196564) (width 0.2) (layer "F.Cu") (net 6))
 (segment (start 178.965936 106.01725) (end 180.126564 106.01725) (width 0.2) (layer "F.Cu") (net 6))
 (segment (start 180.126564 106.01725) (end 182.666564 103.47725) (width 0.2) (layer "F.Cu") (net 6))
 (segment (start 148.36815 105.196564) (end 159.09525 105.196564) (width 0.2) (layer "F.Cu") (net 6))
 (segment (start 187.29725 96.1015) (end 178.576 87.38025) (width 0.2) (layer "F.Cu") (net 6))
 (segment (start 125.46075 89.80425) (end 132.975836 89.80425) (width 0.2) (layer "F.Cu") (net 6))
 (segment (start 161.076564 106.01725) (end 163.546532 103.547282) (width 0.2) (layer "F.Cu") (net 6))
 (segment (start 187.29725 102.656564) (end 187.29725 96.1015) (width 0.2) (layer "F.Cu") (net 6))
 (segment (start 182.666564 103.47725) (end 186.476564 103.47725) (width 0.2) (layer "F.Cu") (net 6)))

